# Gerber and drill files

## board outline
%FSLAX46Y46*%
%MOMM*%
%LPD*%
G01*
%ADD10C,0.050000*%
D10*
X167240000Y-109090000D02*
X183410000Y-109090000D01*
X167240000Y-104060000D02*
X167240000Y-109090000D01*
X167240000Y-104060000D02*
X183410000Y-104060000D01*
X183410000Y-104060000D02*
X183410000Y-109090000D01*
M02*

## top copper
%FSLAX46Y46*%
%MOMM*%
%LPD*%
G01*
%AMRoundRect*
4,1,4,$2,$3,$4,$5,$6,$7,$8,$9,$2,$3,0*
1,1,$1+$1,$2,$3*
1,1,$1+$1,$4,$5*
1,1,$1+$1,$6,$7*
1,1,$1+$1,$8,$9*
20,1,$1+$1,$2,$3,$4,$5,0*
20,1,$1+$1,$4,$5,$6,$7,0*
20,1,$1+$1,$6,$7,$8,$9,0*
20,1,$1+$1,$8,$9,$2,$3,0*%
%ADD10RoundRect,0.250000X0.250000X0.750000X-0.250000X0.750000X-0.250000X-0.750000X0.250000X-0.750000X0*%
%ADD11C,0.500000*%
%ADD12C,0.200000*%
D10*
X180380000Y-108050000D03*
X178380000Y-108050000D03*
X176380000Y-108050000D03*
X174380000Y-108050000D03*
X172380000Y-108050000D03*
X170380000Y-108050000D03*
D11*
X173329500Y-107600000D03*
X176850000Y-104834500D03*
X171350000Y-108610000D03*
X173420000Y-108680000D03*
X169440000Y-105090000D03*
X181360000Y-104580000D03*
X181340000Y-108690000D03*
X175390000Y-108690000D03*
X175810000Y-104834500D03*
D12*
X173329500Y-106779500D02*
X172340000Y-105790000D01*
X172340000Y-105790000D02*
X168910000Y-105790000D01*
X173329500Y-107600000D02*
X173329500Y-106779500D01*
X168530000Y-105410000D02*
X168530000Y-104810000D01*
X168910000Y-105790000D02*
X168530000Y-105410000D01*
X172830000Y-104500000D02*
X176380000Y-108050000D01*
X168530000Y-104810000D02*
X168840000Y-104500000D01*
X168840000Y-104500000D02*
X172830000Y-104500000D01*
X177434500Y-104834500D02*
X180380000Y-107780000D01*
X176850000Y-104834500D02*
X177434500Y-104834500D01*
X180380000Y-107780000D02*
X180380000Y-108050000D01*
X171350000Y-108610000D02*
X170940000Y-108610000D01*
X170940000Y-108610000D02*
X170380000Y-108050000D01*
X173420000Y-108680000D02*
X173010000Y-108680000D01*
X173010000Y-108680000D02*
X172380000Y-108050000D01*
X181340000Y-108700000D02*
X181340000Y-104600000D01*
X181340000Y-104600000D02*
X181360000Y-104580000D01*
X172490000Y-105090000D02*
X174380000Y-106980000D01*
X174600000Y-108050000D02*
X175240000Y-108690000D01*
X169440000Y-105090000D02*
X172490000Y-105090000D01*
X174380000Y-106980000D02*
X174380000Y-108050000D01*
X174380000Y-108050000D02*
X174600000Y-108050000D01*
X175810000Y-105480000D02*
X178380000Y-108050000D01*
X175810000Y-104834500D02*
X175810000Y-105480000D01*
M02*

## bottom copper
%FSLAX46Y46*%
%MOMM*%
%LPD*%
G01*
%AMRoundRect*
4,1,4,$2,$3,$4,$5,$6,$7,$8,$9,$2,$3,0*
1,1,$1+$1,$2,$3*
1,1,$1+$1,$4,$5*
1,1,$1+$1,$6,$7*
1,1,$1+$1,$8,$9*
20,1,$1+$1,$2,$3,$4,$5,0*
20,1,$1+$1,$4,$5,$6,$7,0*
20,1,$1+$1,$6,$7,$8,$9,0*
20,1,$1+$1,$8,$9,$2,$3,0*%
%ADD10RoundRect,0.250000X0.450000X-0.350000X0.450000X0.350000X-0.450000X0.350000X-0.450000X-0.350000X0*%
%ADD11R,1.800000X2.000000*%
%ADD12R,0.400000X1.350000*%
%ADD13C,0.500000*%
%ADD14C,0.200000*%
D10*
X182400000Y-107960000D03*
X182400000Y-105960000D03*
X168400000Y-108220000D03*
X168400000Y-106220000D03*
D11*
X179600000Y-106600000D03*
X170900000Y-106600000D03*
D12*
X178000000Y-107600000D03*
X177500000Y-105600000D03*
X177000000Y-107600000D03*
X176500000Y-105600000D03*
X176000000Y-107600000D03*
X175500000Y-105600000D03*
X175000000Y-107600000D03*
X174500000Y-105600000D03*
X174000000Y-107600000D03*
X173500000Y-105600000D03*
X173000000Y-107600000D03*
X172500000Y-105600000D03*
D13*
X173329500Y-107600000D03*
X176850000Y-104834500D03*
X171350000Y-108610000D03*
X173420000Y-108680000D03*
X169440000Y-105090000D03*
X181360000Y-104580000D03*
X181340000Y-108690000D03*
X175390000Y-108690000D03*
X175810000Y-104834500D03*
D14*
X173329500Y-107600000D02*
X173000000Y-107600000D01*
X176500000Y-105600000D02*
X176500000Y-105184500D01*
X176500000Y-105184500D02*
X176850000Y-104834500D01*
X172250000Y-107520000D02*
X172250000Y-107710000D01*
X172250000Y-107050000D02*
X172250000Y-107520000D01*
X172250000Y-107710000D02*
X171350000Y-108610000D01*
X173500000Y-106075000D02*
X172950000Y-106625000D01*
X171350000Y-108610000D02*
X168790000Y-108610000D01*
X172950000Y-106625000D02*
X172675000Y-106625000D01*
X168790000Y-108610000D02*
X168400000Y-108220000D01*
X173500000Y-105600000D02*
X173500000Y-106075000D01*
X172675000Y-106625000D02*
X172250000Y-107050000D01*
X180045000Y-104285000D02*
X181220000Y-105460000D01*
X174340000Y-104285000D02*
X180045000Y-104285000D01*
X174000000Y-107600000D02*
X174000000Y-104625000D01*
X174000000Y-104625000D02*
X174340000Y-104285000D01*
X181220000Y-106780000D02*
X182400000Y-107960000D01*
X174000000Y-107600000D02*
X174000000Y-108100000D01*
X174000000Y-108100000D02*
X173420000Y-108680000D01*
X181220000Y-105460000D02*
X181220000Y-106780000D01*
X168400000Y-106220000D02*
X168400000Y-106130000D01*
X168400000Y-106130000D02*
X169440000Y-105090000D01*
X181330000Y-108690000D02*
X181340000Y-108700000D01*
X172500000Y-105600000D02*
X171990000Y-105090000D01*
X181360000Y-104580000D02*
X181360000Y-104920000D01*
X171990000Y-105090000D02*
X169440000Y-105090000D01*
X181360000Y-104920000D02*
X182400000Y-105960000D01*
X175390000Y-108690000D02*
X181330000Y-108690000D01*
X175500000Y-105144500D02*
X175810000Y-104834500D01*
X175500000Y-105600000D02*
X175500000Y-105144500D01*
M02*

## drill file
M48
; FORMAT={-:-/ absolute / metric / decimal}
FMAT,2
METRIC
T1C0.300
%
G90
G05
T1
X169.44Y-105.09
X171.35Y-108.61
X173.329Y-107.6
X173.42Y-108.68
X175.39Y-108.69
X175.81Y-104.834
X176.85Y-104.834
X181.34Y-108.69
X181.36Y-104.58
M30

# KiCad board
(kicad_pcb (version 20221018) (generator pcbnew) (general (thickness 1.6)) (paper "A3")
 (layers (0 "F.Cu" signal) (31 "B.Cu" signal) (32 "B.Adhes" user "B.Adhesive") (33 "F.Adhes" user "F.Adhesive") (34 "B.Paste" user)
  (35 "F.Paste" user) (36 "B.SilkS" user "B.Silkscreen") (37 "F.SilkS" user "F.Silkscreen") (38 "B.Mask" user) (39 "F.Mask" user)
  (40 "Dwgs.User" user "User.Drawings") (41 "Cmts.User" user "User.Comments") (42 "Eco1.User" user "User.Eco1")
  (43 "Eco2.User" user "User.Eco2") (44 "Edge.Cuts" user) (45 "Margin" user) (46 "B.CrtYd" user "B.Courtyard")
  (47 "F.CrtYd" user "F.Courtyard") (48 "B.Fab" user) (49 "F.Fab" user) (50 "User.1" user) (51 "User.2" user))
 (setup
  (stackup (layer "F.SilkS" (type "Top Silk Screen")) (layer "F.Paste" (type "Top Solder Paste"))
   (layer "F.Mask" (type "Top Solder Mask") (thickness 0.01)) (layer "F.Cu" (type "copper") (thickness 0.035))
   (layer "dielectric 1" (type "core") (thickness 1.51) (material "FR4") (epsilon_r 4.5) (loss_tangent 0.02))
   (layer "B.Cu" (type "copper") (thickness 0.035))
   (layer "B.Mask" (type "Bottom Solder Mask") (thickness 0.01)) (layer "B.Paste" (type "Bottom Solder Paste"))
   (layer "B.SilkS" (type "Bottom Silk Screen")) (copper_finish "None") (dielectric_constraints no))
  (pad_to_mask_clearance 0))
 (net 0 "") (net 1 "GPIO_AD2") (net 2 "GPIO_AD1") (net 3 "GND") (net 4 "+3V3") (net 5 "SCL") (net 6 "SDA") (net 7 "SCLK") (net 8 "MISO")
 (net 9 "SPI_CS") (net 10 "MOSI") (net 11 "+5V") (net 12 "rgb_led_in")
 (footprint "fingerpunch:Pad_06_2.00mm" (layer "F.Cu") (at 175.38 108.05 180)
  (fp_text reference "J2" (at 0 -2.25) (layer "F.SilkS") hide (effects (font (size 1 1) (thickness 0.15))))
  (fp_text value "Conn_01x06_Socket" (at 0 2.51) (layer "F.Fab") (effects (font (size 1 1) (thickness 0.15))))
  (pad "1" smd roundrect (at -5 0 180) (size 1 2) (layers "F.Cu" "F.Paste" "F.Mask") (roundrect_rratio 0.25) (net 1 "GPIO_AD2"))
  (pad "2" smd roundrect (at -3 0 180) (size 1 2) (layers "F.Cu" "F.Paste" "F.Mask") (roundrect_rratio 0.25) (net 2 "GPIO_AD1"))
  (pad "3" smd roundrect (at -1 0 180) (size 1 2) (layers "F.Cu" "F.Paste" "F.Mask") (roundrect_rratio 0.25) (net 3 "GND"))
  (pad "4" smd roundrect (at 1 0 180) (size 1 2) (layers "F.Cu" "F.Paste" "F.Mask") (roundrect_rratio 0.25) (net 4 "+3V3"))
  (pad "5" smd roundrect (at 3 0 180) (size 1 2) (layers "F.Cu" "F.Paste" "F.Mask") (roundrect_rratio 0.25) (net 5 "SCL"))
  (pad "6" smd roundrect (at 5 0 180) (size 1 2) (layers "F.Cu" "F.Paste" "F.Mask") (roundrect_rratio 0.25) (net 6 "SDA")))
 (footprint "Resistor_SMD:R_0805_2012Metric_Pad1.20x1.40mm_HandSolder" (layer "B.Cu") (at 182.4 106.96 90)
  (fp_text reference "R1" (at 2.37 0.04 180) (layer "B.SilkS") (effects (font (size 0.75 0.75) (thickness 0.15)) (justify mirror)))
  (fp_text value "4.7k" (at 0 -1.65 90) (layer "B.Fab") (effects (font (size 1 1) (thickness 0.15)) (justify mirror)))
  (pad "1" smd roundrect (at -1 0 90) (size 1.2 1.4) (layers "B.Cu" "B.Paste" "B.Mask") (roundrect_rratio 0.2083333333) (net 5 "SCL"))
  (pad "2" smd roundrect (at 1 0 90) (size 1.2 1.4) (layers "B.Cu" "B.Paste" "B.Mask") (roundrect_rratio 0.2083333333) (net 4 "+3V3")))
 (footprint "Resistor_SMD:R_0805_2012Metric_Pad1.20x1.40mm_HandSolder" (layer "B.Cu") (at 168.4 107.22 90)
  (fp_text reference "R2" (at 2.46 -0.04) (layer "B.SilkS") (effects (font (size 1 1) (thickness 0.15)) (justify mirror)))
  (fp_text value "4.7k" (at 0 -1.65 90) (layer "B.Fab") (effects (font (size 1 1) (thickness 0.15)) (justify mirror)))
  (pad "1" smd roundrect (at -1 0 90) (size 1.2 1.4) (layers "B.Cu" "B.Paste" "B.Mask") (roundrect_rratio 0.2083333333) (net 6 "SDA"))
  (pad "2" smd roundrect (at 1 0 90) (size 1.2 1.4) (layers "B.Cu" "B.Paste" "B.Mask") (roundrect_rratio 0.2083333333) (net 4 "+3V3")))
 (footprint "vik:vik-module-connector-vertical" (layer "B.Cu") (at 175.25 106.6 180)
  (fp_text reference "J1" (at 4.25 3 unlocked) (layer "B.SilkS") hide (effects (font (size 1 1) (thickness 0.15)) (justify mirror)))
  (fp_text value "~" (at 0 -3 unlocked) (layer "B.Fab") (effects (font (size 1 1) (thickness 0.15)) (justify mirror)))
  (pad "" smd rect (at -4.35 0 180) (size 1.8 2) (layers "B.Cu" "B.Paste" "B.Mask") (thermal_bridge_angle 45))
  (pad "" smd rect (at 4.35 0 180) (size 1.8 2) (layers "B.Cu" "B.Paste" "B.Mask") (thermal_bridge_angle 45))
  (pad "1" smd rect (at -2.75 -1 180) (size 0.4 1.35) (layers "B.Cu" "B.Paste" "B.Mask") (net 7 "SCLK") (thermal_bridge_angle 45))
  (pad "2" smd rect (at -2.25 1 180) (size 0.4 1.35) (layers "B.Cu" "B.Paste" "B.Mask") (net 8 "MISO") (thermal_bridge_angle 45))
  (pad "3" smd rect (at -1.75 -1 180) (size 0.4 1.35) (layers "B.Cu" "B.Paste" "B.Mask") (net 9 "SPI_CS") (thermal_bridge_angle 45))
  (pad "4" smd rect (at -1.25 1 180) (size 0.4 1.35) (layers "B.Cu" "B.Paste" "B.Mask") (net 1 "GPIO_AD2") (thermal_bridge_angle 45))
  (pad "5" smd rect (at -0.75 -1 180) (size 0.4 1.35) (layers "B.Cu" "B.Paste" "B.Mask") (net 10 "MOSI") (thermal_bridge_angle 45))
  (pad "6" smd rect (at -0.25 1 180) (size 0.4 1.35) (layers "B.Cu" "B.Paste" "B.Mask") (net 2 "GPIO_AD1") (thermal_bridge_angle 45))
  (pad "7" smd rect (at 0.25 -1 180) (size 0.4 1.35) (layers "B.Cu" "B.Paste" "B.Mask") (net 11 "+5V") (thermal_bridge_angle 45))
  (pad "8" smd rect (at 0.75 1 180) (size 0.4 1.35) (layers "B.Cu" "B.Paste" "B.Mask") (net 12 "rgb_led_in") (thermal_bridge_angle 45))
  (pad "9" smd rect (at 1.25 -1 180) (size 0.4 1.35) (layers "B.Cu" "B.Paste" "B.Mask") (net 5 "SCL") (thermal_bridge_angle 45))
  (pad "10" smd rect (at 1.75 1 180) (size 0.4 1.35) (layers "B.Cu" "B.Paste" "B.Mask") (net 6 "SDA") (thermal_bridge_angle 45))
  (pad "11" smd rect (at 2.25 -1 180) (size 0.4 1.35) (layers "B.Cu" "B.Paste" "B.Mask") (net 3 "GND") (thermal_bridge_angle 45))
  (pad "12" smd rect (at 2.75 1 180) (size 0.4 1.35) (layers "B.Cu" "B.Paste" "B.Mask") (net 4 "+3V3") (thermal_bridge_angle 45)))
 (gr_line (start 167.24 109.09) (end 183.41 109.09) (stroke (width 0.05) (type default)) (layer "Edge.Cuts"))
 (gr_line (start 167.24 104.06) (end 167.24 109.09) (stroke (width 0.05) (type default)) (layer "Edge.Cuts"))
 (gr_line (start 167.24 104.06) (end 183.41 104.06) (stroke (width 0.05) (type default)) (layer "Edge.Cuts"))
 (gr_line (start 183.41 104.06) (end 183.41 109.09) (stroke (width 0.05) (type default)) (layer "Edge.Cuts"))
 (segment (start 173.3295 106.7795) (end 172.34 105.79) (width 0.2) (layer "F.Cu") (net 3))
 (segment (start 172.34 105.79) (end 168.91 105.79) (width 0.2) (layer "F.Cu") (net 3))
 (segment (start 173.3295 107.6) (end 173.3295 106.7795) (width 0.2) (layer "F.Cu") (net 3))
 (segment (start 168.53 105.41) (end 168.53 104.81) (width 0.2) (layer "F.Cu") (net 3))
 (segment (start 168.91 105.79) (end 168.53 105.41) (width 0.2) (layer "F.Cu") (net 3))
 (segment (start 172.83 104.5) (end 176.38 108.05) (width 0.2) (layer "F.Cu") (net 3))
 (segment (start 168.53 104.81) (end 168.84 104.5) (width 0.2) (layer "F.Cu") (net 3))
 (segment (start 168.84 104.5) (end 172.83 104.5) (width 0.2) (layer "F.Cu") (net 3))
 (via (at 173.3295 107.6) (size 0.5) (drill 0.3) (layers "F.Cu" "B.Cu") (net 3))
 (segment (start 173.3295 107.6) (end 173 107.6) (width 0.2) (layer "B.Cu") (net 3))
 (segment (start 177.4345 104.8345) (end 180.38 107.78) (width 0.2) (layer "F.Cu") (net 1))
 (segment (start 176.85 104.8345) (end 177.4345 104.8345) (width 0.2) (layer "F.Cu") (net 1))
 (segment (start 180.38 107.78) (end 180.38 108.05) (width 0.2) (layer "F.Cu") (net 1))
 (via (at 176.85 104.8345) (size 0.5) (drill 0.3) (layers "F.Cu" "B.Cu") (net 1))
 (segment (start 176.5 105.6) (end 176.5 105.1845) (width 0.2) (layer "B.Cu") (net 1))
 (segment (start 176.5 105.1845) (end 176.85 104.8345) (width 0.2) (layer "B.Cu") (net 1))
 (segment (start 171.35 108.61) (end 170.94 108.61) (width 0.2) (layer "F.Cu") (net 6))
 (segment (start 170.94 108.61) (end 170.38 108.05) (width 0.2) (layer "F.Cu") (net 6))
 (via (at 171.35 108.61) (size 0.5) (drill 0.3) (layers "F.Cu" "B.Cu") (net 6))
 (segment (start 172.25 107.52) (end 172.25 107.71) (width 0.2) (layer "B.Cu") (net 6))
 (segment (start 172.25 107.05) (end 172.25 107.52) (width 0.2) (layer "B.Cu") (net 6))
 (segment (start 172.25 107.71) (end 171.35 108.61) (width 0.2) (layer "B.Cu") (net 6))
 (segment (start 173.5 106.075) (end 172.95 106.625) (width 0.2) (layer "B.Cu") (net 6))
 (segment (start 171.35 108.61) (end 168.79 108.61) (width 0.2) (layer "B.Cu") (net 6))
 (segment (start 172.95 106.625) (end 172.675 106.625) (width 0.2) (layer "B.Cu") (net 6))
 (segment (start 168.79 108.61) (end 168.4 108.22) (width 0.2) (layer "B.Cu") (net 6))
 (segment (start 173.5 105.6) (end 173.5 106.075) (width 0.2) (layer "B.Cu") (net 6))
 (segment (start 172.675 106.625) (end 172.25 107.05) (width 0.2) (layer "B.Cu") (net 6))
 (segment (start 173.42 108.68) (end 173.01 108.68) (width 0.2) (layer "F.Cu") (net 5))
 (segment (start 173.01 108.68) (end 172.38 108.05) (width 0.2) (layer "F.Cu") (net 5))
 (via (at 173.42 108.68) (size 0.5) (drill 0.3) (layers "F.Cu" "B.Cu") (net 5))
 (segment (start 180.045 104.285) (end 181.22 105.46) (width 0.2) (layer "B.Cu") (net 5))
 (segment (start 174.34 104.285) (end 180.045 104.285) (width 0.2) (layer "B.Cu") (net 5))
 (segment (start 174 107.6) (end 174 104.625) (width 0.2) (layer "B.Cu") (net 5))
 (segment (start 174 104.625) (end 174.34 104.285) (width 0.2) (layer "B.Cu") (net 5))
 (segment (start 181.22 106.78) (end 182.4 107.96) (width 0.2) (layer "B.Cu") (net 5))
 (segment (start 174 107.6) (end 174 108.1) (width 0.2) (layer "B.Cu") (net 5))
 (segment (start 174 108.1) (end 173.42 108.68) (width 0.2) (layer "B.Cu") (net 5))
 (segment (start 181.22 105.46) (end 181.22 106.78) (width 0.2) (layer "B.Cu") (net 5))
 (segment (start 181.34 108.7) (end 181.34 104.6) (width 0.2) (layer "F.Cu") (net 4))
 (segment (start 181.34 104.6) (end 181.36 104.58) (width 0.2) (layer "F.Cu") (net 4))
 (segment (start 172.49 105.09) (end 174.38 106.98) (width 0.2) (layer "F.Cu") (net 4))
 (segment (start 174.6 108.05) (end 175.24 108.69) (width 0.2) (layer "F.Cu") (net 4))
 (segment (start 169.44 105.09) (end 172.49 105.09) (width 0.2) (layer "F.Cu") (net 4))
 (segment (start 174.38 106.98) (end 174.38 108.05) (width 0.2) (layer "F.Cu") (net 4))
 (segment (start 174.38 108.05) (end 174.6 108.05) (width 0.2) (layer "F.Cu") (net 4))
 (via (at 169.44 105.09) (size 0.5) (drill 0.3) (layers "F.Cu" "B.Cu") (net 4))
 (via (at 181.36 104.58) (size 0.5) (drill 0.3) (layers "F.Cu" "B.Cu") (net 4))
 (via (at 181.34 108.69) (size 0.5) (drill 0.3) (layers "F.Cu" "B.Cu") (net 4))
 (via (at 175.39 108.69) (size 0.5) (drill 0.3) (layers "F.Cu" "B.Cu") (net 4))
 (segment (start 168.4 106.22) (end 168.4 106.13) (width 0.2) (layer "B.Cu") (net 4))
 (segment (start 168.4 106.13) (end 169.44 105.09) (width 0.2) (layer "B.Cu") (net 4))
 (segment (start 181.33 108.69) (end 181.34 108.7) (width 0.2) (layer "B.Cu") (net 4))
 (segment (start 172.5 105.6) (end 171.99 105.09) (width 0.2) (layer "B.Cu") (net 4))
 (segment (start 181.36 104.58) (end 181.36 104.92) (width 0.2) (layer "B.Cu") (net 4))
 (segment (start 171.99 105.09) (end 169.44 105.09) (width 0.2) (layer "B.Cu") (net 4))
 (segment (start 181.36 104.92) (end 182.4 105.96) (width 0.2) (layer "B.Cu") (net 4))
 (segment (start 175.39 108.69) (end 181.33 108.69) (width 0.2) (layer "B.Cu") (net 4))
 (segment (start 175.81 105.48) (end 178.38 108.05) (width 0.2) (layer "F.Cu") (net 2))
 (segment (start 175.81 104.8345) (end 175.81 105.48) (width 0.2) (layer "F.Cu") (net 2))
 (via (at 175.81 104.8345) (size 0.5) (drill 0.3) (layers "F.Cu" "B.Cu") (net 2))
 (segment (start 175.5 105.1445) (end 175.81 104.8345) (width 0.2) (layer "B.Cu") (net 2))
 (segment (start 175.5 105.6) (end 175.5 105.1445) (width 0.2) (layer "B.Cu") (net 2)))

